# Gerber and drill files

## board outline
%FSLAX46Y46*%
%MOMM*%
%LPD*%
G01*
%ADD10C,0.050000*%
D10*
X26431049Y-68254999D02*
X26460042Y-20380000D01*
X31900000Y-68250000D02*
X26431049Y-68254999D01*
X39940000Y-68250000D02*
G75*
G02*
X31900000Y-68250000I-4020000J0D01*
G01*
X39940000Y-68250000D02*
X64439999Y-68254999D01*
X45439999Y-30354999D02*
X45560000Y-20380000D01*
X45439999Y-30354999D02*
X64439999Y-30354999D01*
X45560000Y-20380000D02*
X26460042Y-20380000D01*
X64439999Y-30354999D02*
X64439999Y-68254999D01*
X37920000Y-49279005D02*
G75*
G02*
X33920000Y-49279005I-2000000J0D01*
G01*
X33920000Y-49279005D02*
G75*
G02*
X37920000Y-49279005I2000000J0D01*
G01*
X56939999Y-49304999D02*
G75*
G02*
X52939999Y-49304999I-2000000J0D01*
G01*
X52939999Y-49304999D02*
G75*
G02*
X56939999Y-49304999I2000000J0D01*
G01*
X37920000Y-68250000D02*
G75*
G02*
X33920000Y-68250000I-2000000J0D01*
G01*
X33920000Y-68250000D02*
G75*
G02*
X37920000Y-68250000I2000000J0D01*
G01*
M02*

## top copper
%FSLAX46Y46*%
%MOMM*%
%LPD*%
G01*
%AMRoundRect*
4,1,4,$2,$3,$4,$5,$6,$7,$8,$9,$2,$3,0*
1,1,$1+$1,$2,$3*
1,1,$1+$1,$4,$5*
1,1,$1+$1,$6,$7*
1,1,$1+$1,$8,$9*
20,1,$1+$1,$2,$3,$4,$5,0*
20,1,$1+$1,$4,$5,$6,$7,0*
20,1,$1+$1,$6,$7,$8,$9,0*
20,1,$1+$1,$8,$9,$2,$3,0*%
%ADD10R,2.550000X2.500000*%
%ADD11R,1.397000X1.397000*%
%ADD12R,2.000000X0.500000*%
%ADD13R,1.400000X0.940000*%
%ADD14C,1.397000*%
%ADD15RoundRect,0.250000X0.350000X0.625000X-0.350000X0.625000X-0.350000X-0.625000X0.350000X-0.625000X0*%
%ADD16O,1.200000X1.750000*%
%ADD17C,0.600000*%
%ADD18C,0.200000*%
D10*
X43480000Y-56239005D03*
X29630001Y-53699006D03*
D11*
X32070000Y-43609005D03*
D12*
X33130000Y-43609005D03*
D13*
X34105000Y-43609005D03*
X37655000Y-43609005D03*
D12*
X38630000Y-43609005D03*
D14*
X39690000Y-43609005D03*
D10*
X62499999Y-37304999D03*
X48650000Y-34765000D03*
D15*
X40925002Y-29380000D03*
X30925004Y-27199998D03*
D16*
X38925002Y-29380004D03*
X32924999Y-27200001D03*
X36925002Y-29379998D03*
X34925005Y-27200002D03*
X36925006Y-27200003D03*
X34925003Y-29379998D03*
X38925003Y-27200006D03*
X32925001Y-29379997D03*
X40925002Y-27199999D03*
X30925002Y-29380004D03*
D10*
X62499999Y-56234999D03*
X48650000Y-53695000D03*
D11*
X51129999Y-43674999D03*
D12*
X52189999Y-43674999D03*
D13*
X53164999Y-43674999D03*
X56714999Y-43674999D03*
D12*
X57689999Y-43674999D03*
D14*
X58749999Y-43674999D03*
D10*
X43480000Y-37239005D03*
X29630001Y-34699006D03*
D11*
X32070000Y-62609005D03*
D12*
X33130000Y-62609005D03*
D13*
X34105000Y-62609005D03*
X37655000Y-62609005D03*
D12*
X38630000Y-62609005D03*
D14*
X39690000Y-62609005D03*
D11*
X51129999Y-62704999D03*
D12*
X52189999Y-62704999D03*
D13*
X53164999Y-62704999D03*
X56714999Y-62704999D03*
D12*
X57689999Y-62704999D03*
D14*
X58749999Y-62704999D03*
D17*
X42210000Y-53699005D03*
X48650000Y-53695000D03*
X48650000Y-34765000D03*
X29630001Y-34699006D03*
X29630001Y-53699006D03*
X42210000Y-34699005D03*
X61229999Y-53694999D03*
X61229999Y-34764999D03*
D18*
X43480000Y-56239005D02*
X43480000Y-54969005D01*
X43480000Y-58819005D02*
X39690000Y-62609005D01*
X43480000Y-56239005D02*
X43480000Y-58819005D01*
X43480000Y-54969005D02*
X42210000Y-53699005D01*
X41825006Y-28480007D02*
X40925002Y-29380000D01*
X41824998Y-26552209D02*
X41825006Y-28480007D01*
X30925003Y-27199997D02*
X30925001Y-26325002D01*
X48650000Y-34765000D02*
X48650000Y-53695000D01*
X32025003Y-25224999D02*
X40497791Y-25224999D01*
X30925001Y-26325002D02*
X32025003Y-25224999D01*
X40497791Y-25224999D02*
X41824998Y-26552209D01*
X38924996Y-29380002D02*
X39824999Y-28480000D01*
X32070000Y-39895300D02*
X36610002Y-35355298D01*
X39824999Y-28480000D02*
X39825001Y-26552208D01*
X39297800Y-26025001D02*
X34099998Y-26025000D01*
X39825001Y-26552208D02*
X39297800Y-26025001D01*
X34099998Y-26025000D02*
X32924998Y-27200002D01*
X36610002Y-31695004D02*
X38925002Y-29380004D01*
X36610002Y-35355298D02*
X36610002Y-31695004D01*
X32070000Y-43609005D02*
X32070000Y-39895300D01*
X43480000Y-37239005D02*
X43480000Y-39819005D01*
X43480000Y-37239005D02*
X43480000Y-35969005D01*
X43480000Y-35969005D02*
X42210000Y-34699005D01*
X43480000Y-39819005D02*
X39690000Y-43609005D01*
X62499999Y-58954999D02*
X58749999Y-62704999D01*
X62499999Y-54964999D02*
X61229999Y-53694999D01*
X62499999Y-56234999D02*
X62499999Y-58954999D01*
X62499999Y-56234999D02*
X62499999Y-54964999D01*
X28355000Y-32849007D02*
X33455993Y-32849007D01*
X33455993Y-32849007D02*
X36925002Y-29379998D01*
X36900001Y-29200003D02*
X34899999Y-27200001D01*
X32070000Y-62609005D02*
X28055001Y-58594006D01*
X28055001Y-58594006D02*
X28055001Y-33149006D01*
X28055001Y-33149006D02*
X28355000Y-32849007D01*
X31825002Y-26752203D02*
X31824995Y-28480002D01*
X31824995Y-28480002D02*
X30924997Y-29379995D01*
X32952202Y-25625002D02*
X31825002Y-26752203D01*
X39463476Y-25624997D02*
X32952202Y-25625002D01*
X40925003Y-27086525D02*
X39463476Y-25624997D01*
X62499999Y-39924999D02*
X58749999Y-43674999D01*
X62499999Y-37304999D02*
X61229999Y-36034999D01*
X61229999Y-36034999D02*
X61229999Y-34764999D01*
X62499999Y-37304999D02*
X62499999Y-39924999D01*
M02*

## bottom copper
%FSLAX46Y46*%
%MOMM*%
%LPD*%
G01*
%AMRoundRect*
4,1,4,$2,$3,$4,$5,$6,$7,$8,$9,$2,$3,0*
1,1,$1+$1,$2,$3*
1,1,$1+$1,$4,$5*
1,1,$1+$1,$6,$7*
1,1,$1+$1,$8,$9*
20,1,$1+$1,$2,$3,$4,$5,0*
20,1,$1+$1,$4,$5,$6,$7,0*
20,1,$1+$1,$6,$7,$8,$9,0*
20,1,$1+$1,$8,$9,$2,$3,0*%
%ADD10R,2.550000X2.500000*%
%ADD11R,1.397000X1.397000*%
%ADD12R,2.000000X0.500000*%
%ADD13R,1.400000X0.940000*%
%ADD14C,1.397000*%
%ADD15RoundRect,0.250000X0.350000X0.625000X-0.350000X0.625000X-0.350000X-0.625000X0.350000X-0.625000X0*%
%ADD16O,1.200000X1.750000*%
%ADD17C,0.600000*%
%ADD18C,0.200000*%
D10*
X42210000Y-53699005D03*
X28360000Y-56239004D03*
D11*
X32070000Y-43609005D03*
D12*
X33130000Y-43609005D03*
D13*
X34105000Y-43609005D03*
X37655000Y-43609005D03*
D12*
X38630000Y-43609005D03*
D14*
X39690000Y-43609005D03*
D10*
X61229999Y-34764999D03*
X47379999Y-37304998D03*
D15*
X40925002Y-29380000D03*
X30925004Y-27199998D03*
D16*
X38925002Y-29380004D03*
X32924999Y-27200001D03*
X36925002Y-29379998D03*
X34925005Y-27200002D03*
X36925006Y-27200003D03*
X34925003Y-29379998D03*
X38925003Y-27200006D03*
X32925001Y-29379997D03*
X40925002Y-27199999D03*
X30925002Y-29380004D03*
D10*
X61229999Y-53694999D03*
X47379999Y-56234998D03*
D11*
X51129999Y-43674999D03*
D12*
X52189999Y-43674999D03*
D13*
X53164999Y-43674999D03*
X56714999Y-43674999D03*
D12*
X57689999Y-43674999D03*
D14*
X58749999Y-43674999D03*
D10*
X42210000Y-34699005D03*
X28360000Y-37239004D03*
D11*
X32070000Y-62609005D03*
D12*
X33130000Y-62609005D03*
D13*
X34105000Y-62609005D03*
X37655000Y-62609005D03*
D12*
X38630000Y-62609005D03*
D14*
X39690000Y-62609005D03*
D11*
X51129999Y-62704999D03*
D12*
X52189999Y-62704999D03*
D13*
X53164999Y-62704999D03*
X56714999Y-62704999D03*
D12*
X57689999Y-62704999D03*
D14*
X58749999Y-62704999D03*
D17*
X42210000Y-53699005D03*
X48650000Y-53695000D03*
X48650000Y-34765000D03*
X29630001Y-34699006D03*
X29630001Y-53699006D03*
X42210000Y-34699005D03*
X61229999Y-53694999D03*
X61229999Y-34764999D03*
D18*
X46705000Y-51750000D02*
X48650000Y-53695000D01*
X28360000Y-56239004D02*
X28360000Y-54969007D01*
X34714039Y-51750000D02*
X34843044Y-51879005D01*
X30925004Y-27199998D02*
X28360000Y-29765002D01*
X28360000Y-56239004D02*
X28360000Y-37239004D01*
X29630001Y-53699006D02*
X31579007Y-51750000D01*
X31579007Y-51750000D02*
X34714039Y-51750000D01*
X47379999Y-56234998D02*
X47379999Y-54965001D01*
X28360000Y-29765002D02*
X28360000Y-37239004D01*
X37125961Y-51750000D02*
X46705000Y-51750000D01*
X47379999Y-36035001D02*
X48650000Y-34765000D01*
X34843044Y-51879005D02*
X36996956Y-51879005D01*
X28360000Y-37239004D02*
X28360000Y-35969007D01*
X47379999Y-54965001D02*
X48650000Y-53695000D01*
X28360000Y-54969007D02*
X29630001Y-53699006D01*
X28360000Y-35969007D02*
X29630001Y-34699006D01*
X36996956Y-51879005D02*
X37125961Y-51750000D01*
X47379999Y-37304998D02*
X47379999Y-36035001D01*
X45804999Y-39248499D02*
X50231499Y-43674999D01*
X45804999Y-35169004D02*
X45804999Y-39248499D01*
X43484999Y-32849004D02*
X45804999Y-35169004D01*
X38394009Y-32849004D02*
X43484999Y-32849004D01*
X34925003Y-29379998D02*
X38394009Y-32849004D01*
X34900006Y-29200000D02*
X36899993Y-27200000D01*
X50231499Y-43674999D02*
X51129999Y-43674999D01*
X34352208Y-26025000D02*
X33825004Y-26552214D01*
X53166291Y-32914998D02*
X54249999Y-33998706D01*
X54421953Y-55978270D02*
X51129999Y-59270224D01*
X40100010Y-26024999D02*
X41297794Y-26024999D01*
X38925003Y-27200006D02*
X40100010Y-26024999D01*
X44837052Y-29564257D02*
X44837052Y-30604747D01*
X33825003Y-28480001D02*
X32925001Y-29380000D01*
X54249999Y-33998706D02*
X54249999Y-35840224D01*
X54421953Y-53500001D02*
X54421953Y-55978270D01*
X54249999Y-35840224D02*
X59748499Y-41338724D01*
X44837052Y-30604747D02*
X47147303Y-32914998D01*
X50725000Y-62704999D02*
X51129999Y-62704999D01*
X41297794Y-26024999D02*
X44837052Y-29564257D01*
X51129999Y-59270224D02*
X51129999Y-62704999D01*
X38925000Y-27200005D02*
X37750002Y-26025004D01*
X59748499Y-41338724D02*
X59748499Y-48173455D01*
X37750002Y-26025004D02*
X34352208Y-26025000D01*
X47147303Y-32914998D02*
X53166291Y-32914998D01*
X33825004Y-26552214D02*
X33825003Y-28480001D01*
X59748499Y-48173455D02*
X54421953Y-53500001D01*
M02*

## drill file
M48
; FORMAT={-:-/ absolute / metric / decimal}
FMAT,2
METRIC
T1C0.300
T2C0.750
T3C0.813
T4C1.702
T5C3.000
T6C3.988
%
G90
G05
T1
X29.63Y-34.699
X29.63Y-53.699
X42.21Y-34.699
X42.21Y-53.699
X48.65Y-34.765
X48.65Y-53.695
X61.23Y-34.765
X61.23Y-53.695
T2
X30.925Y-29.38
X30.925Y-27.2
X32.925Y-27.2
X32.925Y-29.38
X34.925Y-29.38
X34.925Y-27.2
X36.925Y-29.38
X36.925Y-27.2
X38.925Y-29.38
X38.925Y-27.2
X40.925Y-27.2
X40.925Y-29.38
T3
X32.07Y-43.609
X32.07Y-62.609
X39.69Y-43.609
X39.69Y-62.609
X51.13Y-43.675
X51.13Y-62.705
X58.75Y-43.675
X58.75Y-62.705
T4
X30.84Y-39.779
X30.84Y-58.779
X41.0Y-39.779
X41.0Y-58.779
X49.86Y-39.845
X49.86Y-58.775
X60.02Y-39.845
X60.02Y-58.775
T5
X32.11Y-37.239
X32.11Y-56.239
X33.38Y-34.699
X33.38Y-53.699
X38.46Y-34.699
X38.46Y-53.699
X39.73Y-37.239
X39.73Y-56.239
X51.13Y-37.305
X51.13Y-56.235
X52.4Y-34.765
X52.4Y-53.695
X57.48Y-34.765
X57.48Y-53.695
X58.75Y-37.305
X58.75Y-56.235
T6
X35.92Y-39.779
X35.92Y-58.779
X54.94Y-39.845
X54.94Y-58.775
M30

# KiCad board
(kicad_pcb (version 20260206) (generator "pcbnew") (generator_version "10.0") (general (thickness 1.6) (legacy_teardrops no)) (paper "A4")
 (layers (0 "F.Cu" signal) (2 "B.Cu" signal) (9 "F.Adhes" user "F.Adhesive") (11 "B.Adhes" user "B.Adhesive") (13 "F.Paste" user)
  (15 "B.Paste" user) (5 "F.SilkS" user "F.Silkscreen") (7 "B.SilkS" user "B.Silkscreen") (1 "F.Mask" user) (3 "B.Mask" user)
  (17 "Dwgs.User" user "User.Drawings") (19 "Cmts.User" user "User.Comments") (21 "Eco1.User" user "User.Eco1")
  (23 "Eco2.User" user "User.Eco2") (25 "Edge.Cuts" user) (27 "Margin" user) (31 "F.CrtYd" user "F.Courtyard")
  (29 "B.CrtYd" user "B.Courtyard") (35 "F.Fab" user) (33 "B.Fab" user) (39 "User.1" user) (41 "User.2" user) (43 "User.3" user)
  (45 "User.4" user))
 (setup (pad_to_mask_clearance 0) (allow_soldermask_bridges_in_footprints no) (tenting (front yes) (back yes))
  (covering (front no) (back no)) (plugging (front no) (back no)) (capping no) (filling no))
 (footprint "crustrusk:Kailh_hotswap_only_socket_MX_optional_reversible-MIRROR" (layer "F.Cu") (at 35.92 58.779005)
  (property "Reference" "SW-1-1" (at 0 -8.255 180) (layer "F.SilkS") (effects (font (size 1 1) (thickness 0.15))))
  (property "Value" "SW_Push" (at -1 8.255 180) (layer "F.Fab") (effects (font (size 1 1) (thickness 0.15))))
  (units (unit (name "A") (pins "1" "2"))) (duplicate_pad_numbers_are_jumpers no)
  (pad "" np_thru_hole circle (at -5.08 0) (size 1.7018 1.7018) (drill 1.7018) (layers "*.Cu" "*.Mask"))
  (pad "" np_thru_hole circle (at -3.81 -2.54 180) (size 3 3) (drill 3) (layers "*.Cu" "*.Mask"))
  (pad "" np_thru_hole circle (at -2.54 -5.079998) (size 3 3) (drill 3) (layers "*.Cu" "*.Mask"))
  (pad "" np_thru_hole circle (at 0 0) (size 3.9878 3.9878) (drill 3.9878) (layers "*.Cu" "*.Mask"))
  (pad "" np_thru_hole circle (at 2.540002 -5.080001 180) (size 3 3) (drill 3) (layers "*.Cu" "*.Mask"))
  (pad "" np_thru_hole circle (at 3.81 -2.54) (size 3 3) (drill 3) (layers "*.Cu" "*.Mask"))
  (pad "" np_thru_hole circle (at 5.08 0) (size 1.7018 1.7018) (drill 1.7018) (layers "*.Cu" "*.Mask"))
  (pad "1" smd rect (at 6.29 -5.08 180) (size 2.55 2.5) (layers "B.Cu" "B.Mask" "B.Paste") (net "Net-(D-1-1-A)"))
  (pad "1" smd rect (at 7.56 -2.54) (size 2.55 2.5) (layers "F.Cu" "F.Mask" "F.Paste") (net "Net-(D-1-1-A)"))
  (pad "2" smd rect (at -7.56 -2.540001 180) (size 2.55 2.5) (layers "B.Cu" "B.Mask" "B.Paste") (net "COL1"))
  (pad "2" smd rect (at -6.289999 -5.079999) (size 2.55 2.5) (layers "F.Cu" "F.Mask" "F.Paste") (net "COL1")))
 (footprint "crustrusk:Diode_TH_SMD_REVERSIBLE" (layer "F.Cu") (at 35.88 43.609005)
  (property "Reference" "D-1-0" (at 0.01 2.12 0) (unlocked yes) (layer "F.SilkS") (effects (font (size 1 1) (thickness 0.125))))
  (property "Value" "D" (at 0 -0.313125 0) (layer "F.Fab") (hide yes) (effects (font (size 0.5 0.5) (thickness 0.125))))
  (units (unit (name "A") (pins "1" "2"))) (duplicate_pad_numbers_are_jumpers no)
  (pad "1" thru_hole rect (at -3.81 0) (size 1.397 1.397) (drill 0.8128) (layers "*.Cu" "*.Mask") (remove_unused_layers no) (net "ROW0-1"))
  (pad "1" smd rect (at -2.75 0 180) (size 2 0.5) (layers "F.Cu") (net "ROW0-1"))
  (pad "1" smd rect (at -2.75 0) (size 2 0.5) (layers "B.Cu") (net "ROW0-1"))
  (pad "1" smd rect (at -1.775 0 180) (size 1.4 0.94) (layers "F.Cu" "F.Mask" "F.Paste") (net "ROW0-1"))
  (pad "1" smd rect (at -1.775 0) (size 1.4 0.94) (layers "B.Cu" "B.Mask" "B.Paste") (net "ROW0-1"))
  (pad "2" smd rect (at 1.775 0 180) (size 1.4 0.94) (layers "F.Cu" "F.Mask" "F.Paste") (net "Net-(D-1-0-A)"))
  (pad "2" smd rect (at 1.775 0) (size 1.4 0.94) (layers "B.Cu" "B.Mask" "B.Paste") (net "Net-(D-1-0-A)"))
  (pad "2" smd rect (at 2.75 0 180) (size 2 0.5) (layers "F.Cu") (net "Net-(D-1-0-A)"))
  (pad "2" smd rect (at 2.75 0) (size 2 0.5) (layers "B.Cu") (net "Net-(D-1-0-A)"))
  (pad "2" thru_hole circle (at 3.81 0) (size 1.397 1.397) (drill 0.8128) (layers "*.Cu" "*.Mask") (remove_unused_layers no)
   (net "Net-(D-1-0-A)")))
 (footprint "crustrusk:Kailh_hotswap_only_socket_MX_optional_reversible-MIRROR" (layer "F.Cu") (at 54.939999 39.844999)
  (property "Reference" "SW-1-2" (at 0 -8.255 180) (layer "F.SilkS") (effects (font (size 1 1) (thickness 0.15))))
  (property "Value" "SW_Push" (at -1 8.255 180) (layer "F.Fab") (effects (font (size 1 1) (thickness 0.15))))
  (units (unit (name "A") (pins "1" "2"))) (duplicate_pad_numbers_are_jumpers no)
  (pad "" np_thru_hole circle (at -5.08 0) (size 1.7018 1.7018) (drill 1.7018) (layers "*.Cu" "*.Mask"))
  (pad "" np_thru_hole circle (at -3.81 -2.54 180) (size 3 3) (drill 3) (layers "*.Cu" "*.Mask"))
  (pad "" np_thru_hole circle (at -2.54 -5.079998) (size 3 3) (drill 3) (layers "*.Cu" "*.Mask"))
  (pad "" np_thru_hole circle (at 0 0) (size 3.9878 3.9878) (drill 3.9878) (layers "*.Cu" "*.Mask"))
  (pad "" np_thru_hole circle (at 2.540002 -5.080001 180) (size 3 3) (drill 3) (layers "*.Cu" "*.Mask"))
  (pad "" np_thru_hole circle (at 3.81 -2.54) (size 3 3) (drill 3) (layers "*.Cu" "*.Mask"))
  (pad "" np_thru_hole circle (at 5.08 0) (size 1.7018 1.7018) (drill 1.7018) (layers "*.Cu" "*.Mask"))
  (pad "1" smd rect (at 6.29 -5.08 180) (size 2.55 2.5) (layers "B.Cu" "B.Mask" "B.Paste") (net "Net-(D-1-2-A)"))
  (pad "1" smd rect (at 7.56 -2.54) (size 2.55 2.5) (layers "F.Cu" "F.Mask" "F.Paste") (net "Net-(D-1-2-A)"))
  (pad "2" smd rect (at -7.56 -2.540001 180) (size 2.55 2.5) (layers "B.Cu" "B.Mask" "B.Paste") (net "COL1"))
  (pad "2" smd rect (at -6.289999 -5.079999) (size 2.55 2.5) (layers "F.Cu" "F.Mask" "F.Paste") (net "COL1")))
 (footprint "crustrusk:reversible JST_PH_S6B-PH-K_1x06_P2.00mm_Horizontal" (layer "F.Cu") (at 40.925002 29.38 180)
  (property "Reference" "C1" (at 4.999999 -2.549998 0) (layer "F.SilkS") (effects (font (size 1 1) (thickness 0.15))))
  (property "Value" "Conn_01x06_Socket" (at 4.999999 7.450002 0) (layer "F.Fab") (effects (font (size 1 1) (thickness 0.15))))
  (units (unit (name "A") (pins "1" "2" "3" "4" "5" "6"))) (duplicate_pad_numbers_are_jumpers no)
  (pad "1" thru_hole roundrect (at 0 0 180) (size 1.2 1.75) (drill 0.75) (layers "*.Cu" "*.Mask") (remove_unused_layers no)
   (roundrect_rratio 0.208333) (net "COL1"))
  (pad "1" thru_hole roundrect (at 9.999998 2.180002 180) (size 1.2 1.75) (drill 0.75) (layers "*.Cu" "*.Mask") (remove_unused_layers no)
   (roundrect_rratio 0.208333) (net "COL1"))
  (pad "2" thru_hole oval (at 2 -0.000004 180) (size 1.2 1.75) (drill 0.75) (layers "*.Cu" "*.Mask") (remove_unused_layers no)
   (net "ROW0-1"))
  (pad "2" thru_hole oval (at 8.000003 2.179999 180) (size 1.2 1.75) (drill 0.75) (layers "*.Cu" "*.Mask") (remove_unused_layers no)
   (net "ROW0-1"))
  (pad "3" thru_hole oval (at 4 0.000002 180) (size 1.2 1.75) (drill 0.75) (layers "*.Cu" "*.Mask") (remove_unused_layers no) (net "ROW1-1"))
  (pad "3" thru_hole oval (at 5.999997 2.179998 180) (size 1.2 1.75) (drill 0.75) (layers "*.Cu" "*.Mask") (remove_unused_layers no)
   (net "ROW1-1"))
  (pad "4" thru_hole oval (at 3.999996 2.179997 180) (size 1.2 1.75) (drill 0.75) (layers "*.Cu" "*.Mask") (remove_unused_layers no)
   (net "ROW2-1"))
  (pad "4" thru_hole oval (at 5.999999 0.000002 180) (size 1.2 1.75) (drill 0.75) (layers "*.Cu" "*.Mask") (remove_unused_layers no)
   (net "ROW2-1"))
  (pad "5" thru_hole oval (at 1.999999 2.179994 180) (size 1.2 1.75) (drill 0.75) (layers "*.Cu" "*.Mask") (remove_unused_layers no)
   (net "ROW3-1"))
  (pad "5" thru_hole oval (at 8.000001 0.000003 180) (size 1.2 1.75) (drill 0.75) (layers "*.Cu" "*.Mask") (remove_unused_layers no)
   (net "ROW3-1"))
  (pad "6" thru_hole oval (at 0 2.180001 180) (size 1.2 1.75) (drill 0.75) (layers "*.Cu" "*.Mask") (remove_unused_layers no) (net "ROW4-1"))
  (pad "6" thru_hole oval (at 10 -0.000004 180) (size 1.2 1.75) (drill 0.75) (layers "*.Cu" "*.Mask") (remove_unused_layers no)
   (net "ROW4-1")))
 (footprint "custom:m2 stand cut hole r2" (layer "F.Cu") (at 35.92 49.279005)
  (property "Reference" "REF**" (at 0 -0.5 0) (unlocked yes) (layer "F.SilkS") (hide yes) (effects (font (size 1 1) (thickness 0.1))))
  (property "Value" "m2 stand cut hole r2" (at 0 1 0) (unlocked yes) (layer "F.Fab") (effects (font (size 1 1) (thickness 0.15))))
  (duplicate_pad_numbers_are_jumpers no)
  (fp_circle (center 0 0) (end 2 0) (stroke (width 0.05) (type default)) (fill no) (layer "Edge.Cuts")))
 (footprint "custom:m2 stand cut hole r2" (layer "F.Cu") (at 54.939999 49.304999)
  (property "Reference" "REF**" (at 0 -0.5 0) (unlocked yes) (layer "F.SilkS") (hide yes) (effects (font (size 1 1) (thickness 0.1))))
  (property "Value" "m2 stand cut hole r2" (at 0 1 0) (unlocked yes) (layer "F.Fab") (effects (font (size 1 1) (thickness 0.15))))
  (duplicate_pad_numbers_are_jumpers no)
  (fp_circle (center 0 0) (end 2 0) (stroke (width 0.05) (type default)) (fill no) (layer "Edge.Cuts")))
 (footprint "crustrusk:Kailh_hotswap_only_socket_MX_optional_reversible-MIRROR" (layer "F.Cu") (at 54.939999 58.774999)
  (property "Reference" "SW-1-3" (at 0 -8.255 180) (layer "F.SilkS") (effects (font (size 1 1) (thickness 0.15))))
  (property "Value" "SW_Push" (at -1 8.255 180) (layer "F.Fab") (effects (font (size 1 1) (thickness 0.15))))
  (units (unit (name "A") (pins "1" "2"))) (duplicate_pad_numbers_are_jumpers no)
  (pad "" np_thru_hole circle (at -5.08 0) (size 1.7018 1.7018) (drill 1.7018) (layers "*.Cu" "*.Mask"))
  (pad "" np_thru_hole circle (at -3.81 -2.54 180) (size 3 3) (drill 3) (layers "*.Cu" "*.Mask"))
  (pad "" np_thru_hole circle (at -2.54 -5.079998) (size 3 3) (drill 3) (layers "*.Cu" "*.Mask"))
  (pad "" np_thru_hole circle (at 0 0) (size 3.9878 3.9878) (drill 3.9878) (layers "*.Cu" "*.Mask"))
  (pad "" np_thru_hole circle (at 2.540002 -5.080001 180) (size 3 3) (drill 3) (layers "*.Cu" "*.Mask"))
  (pad "" np_thru_hole circle (at 3.81 -2.54) (size 3 3) (drill 3) (layers "*.Cu" "*.Mask"))
  (pad "" np_thru_hole circle (at 5.08 0) (size 1.7018 1.7018) (drill 1.7018) (layers "*.Cu" "*.Mask"))
  (pad "1" smd rect (at 6.29 -5.08 180) (size 2.55 2.5) (layers "B.Cu" "B.Mask" "B.Paste") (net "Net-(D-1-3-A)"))
  (pad "1" smd rect (at 7.56 -2.54) (size 2.55 2.5) (layers "F.Cu" "F.Mask" "F.Paste") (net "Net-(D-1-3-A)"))
  (pad "2" smd rect (at -7.56 -2.540001 180) (size 2.55 2.5) (layers "B.Cu" "B.Mask" "B.Paste") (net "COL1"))
  (pad "2" smd rect (at -6.289999 -5.079999) (size 2.55 2.5) (layers "F.Cu" "F.Mask" "F.Paste") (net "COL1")))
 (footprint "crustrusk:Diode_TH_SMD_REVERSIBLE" (layer "F.Cu") (at 54.939999 43.674999)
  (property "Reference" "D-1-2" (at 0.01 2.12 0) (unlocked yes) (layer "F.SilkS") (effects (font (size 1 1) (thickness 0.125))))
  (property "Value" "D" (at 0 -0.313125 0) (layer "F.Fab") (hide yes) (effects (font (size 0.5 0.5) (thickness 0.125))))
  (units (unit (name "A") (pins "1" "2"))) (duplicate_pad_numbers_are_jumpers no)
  (pad "1" thru_hole rect (at -3.81 0) (size 1.397 1.397) (drill 0.8128) (layers "*.Cu" "*.Mask") (remove_unused_layers no) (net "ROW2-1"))
  (pad "1" smd rect (at -2.75 0 180) (size 2 0.5) (layers "F.Cu") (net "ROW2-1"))
  (pad "1" smd rect (at -2.75 0) (size 2 0.5) (layers "B.Cu") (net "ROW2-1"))
  (pad "1" smd rect (at -1.775 0 180) (size 1.4 0.94) (layers "F.Cu" "F.Mask" "F.Paste") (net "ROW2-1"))
  (pad "1" smd rect (at -1.775 0) (size 1.4 0.94) (layers "B.Cu" "B.Mask" "B.Paste") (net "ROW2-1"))
  (pad "2" smd rect (at 1.775 0 180) (size 1.4 0.94) (layers "F.Cu" "F.Mask" "F.Paste") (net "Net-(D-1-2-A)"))
  (pad "2" smd rect (at 1.775 0) (size 1.4 0.94) (layers "B.Cu" "B.Mask" "B.Paste") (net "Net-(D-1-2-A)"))
  (pad "2" smd rect (at 2.75 0 180) (size 2 0.5) (layers "F.Cu") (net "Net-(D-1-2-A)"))
  (pad "2" smd rect (at 2.75 0) (size 2 0.5) (layers "B.Cu") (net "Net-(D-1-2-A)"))
  (pad "2" thru_hole circle (at 3.81 0) (size 1.397 1.397) (drill 0.8128) (layers "*.Cu" "*.Mask") (remove_unused_layers no)
   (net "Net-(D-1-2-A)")))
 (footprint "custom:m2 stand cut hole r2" (layer "F.Cu") (at 35.92 68.25)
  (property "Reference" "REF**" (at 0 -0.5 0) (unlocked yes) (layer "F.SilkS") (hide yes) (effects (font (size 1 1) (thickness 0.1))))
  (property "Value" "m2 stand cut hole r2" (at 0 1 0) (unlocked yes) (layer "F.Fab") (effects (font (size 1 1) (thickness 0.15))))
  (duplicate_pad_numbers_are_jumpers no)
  (fp_circle (center 0 0) (end 2 0) (stroke (width 0.05) (type default)) (fill no) (layer "Edge.Cuts")))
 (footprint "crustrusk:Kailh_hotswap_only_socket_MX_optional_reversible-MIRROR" (layer "F.Cu") (at 35.92 39.779005)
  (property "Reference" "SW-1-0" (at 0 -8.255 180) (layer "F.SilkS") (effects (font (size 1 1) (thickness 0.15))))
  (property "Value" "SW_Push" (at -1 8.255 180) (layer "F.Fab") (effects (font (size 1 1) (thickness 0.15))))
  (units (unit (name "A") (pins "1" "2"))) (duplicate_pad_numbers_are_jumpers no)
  (pad "" np_thru_hole circle (at -5.08 0) (size 1.7018 1.7018) (drill 1.7018) (layers "*.Cu" "*.Mask"))
  (pad "" np_thru_hole circle (at -3.81 -2.54 180) (size 3 3) (drill 3) (layers "*.Cu" "*.Mask"))
  (pad "" np_thru_hole circle (at -2.54 -5.079998) (size 3 3) (drill 3) (layers "*.Cu" "*.Mask"))
  (pad "" np_thru_hole circle (at 0 0) (size 3.9878 3.9878) (drill 3.9878) (layers "*.Cu" "*.Mask"))
  (pad "" np_thru_hole circle (at 2.540002 -5.080001 180) (size 3 3) (drill 3) (layers "*.Cu" "*.Mask"))
  (pad "" np_thru_hole circle (at 3.81 -2.54) (size 3 3) (drill 3) (layers "*.Cu" "*.Mask"))
  (pad "" np_thru_hole circle (at 5.08 0) (size 1.7018 1.7018) (drill 1.7018) (layers "*.Cu" "*.Mask"))
  (pad "1" smd rect (at 6.29 -5.08 180) (size 2.55 2.5) (layers "B.Cu" "B.Mask" "B.Paste") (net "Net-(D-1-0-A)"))
  (pad "1" smd rect (at 7.56 -2.54) (size 2.55 2.5) (layers "F.Cu" "F.Mask" "F.Paste") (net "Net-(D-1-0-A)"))
  (pad "2" smd rect (at -7.56 -2.540001 180) (size 2.55 2.5) (layers "B.Cu" "B.Mask" "B.Paste") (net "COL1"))
  (pad "2" smd rect (at -6.289999 -5.079999) (size 2.55 2.5) (layers "F.Cu" "F.Mask" "F.Paste") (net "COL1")))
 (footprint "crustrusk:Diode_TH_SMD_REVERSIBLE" (layer "F.Cu") (at 35.88 62.609005)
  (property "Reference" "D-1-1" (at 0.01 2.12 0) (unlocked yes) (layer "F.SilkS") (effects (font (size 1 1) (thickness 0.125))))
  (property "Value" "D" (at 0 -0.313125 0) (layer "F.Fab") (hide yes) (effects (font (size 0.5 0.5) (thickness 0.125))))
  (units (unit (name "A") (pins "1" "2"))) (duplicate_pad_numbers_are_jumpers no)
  (pad "1" thru_hole rect (at -3.81 0) (size 1.397 1.397) (drill 0.8128) (layers "*.Cu" "*.Mask") (remove_unused_layers no) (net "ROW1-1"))
  (pad "1" smd rect (at -2.75 0 180) (size 2 0.5) (layers "F.Cu") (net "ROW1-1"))
  (pad "1" smd rect (at -2.75 0) (size 2 0.5) (layers "B.Cu") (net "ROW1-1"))
  (pad "1" smd rect (at -1.775 0 180) (size 1.4 0.94) (layers "F.Cu" "F.Mask" "F.Paste") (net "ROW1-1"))
  (pad "1" smd rect (at -1.775 0) (size 1.4 0.94) (layers "B.Cu" "B.Mask" "B.Paste") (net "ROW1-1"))
  (pad "2" smd rect (at 1.775 0 180) (size 1.4 0.94) (layers "F.Cu" "F.Mask" "F.Paste") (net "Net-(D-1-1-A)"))
  (pad "2" smd rect (at 1.775 0) (size 1.4 0.94) (layers "B.Cu" "B.Mask" "B.Paste") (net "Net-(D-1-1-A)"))
  (pad "2" smd rect (at 2.75 0 180) (size 2 0.5) (layers "F.Cu") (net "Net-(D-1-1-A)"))
  (pad "2" smd rect (at 2.75 0) (size 2 0.5) (layers "B.Cu") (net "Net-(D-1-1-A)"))
  (pad "2" thru_hole circle (at 3.81 0) (size 1.397 1.397) (drill 0.8128) (layers "*.Cu" "*.Mask") (remove_unused_layers no)
   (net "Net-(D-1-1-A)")))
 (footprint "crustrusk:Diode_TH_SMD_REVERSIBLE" (layer "F.Cu") (at 54.939999 62.704999)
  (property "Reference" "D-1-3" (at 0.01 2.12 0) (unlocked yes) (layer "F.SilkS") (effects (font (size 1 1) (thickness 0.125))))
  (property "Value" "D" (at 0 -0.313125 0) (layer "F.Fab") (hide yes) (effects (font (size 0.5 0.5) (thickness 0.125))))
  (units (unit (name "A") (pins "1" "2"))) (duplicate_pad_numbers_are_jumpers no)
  (pad "1" thru_hole rect (at -3.81 0) (size 1.397 1.397) (drill 0.8128) (layers "*.Cu" "*.Mask") (remove_unused_layers no) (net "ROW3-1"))
  (pad "1" smd rect (at -2.75 0 180) (size 2 0.5) (layers "F.Cu") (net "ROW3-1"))
  (pad "1" smd rect (at -2.75 0) (size 2 0.5) (layers "B.Cu") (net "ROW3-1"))
  (pad "1" smd rect (at -1.775 0 180) (size 1.4 0.94) (layers "F.Cu" "F.Mask" "F.Paste") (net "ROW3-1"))
  (pad "1" smd rect (at -1.775 0) (size 1.4 0.94) (layers "B.Cu" "B.Mask" "B.Paste") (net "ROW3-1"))
  (pad "2" smd rect (at 1.775 0 180) (size 1.4 0.94) (layers "F.Cu" "F.Mask" "F.Paste") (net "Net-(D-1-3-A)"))
  (pad "2" smd rect (at 1.775 0) (size 1.4 0.94) (layers "B.Cu" "B.Mask" "B.Paste") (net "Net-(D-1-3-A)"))
  (pad "2" smd rect (at 2.75 0 180) (size 2 0.5) (layers "F.Cu") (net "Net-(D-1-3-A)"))
  (pad "2" smd rect (at 2.75 0) (size 2 0.5) (layers "B.Cu") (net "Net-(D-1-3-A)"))
  (pad "2" thru_hole circle (at 3.81 0) (size 1.397 1.397) (drill 0.8128) (layers "*.Cu" "*.Mask") (remove_unused_layers no)
   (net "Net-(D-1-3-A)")))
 (gr_line (start 26.431049 68.254999) (end 26.460042 20.38) (stroke (width 0.05) (type default)) (layer "Edge.Cuts"))
 (gr_line (start 31.9 68.25) (end 26.431049 68.254999) (stroke (width 0.05) (type default)) (layer "Edge.Cuts"))
 (gr_arc (start 39.94 68.25) (mid 35.92 72.27) (end 31.9 68.25) (stroke (width 0.05) (type default)) (layer "Edge.Cuts"))
 (gr_line (start 39.94 68.25) (end 64.439999 68.254999) (stroke (width 0.05) (type default)) (layer "Edge.Cuts"))
 (gr_line (start 45.439999 30.354999) (end 45.56 20.38) (stroke (width 0.05) (type default)) (layer "Edge.Cuts"))
 (gr_line (start 45.439999 30.354999) (end 64.439999 30.354999) (stroke (width 0.05) (type default)) (layer "Edge.Cuts"))
 (gr_line (start 45.56 20.38) (end 26.460042 20.38) (stroke (width 0.05) (type default)) (layer "Edge.Cuts"))
 (gr_line (start 64.439999 30.354999) (end 64.439999 68.254999) (stroke (width 0.05) (type default)) (layer "Edge.Cuts"))
 (segment (start 43.48 56.239005) (end 43.48 54.969005) (width 0.2) (layer "F.Cu") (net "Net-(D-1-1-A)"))
 (segment (start 43.48 58.819005) (end 39.69 62.609005) (width 0.2) (layer "F.Cu") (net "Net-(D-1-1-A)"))
 (segment (start 43.48 56.239005) (end 43.48 58.819005) (width 0.2) (layer "F.Cu") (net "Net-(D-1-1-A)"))
 (segment (start 43.48 54.969005) (end 42.21 53.699005) (width 0.2) (layer "F.Cu") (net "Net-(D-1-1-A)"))
 (via (at 42.21 53.699005) (size 0.6) (drill 0.3) (layers "F.Cu" "B.Cu") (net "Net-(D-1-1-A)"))
 (segment (start 41.825006 28.480007) (end 40.925002 29.38) (width 0.2) (layer "F.Cu") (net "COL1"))
 (segment (start 41.824998 26.552209) (end 41.825006 28.480007) (width 0.2) (layer "F.Cu") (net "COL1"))
 (segment (start 30.925003 27.199997) (end 30.925001 26.325002) (width 0.2) (layer "F.Cu") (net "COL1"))
 (segment (start 48.65 34.765) (end 48.65 53.695) (width 0.2) (layer "F.Cu") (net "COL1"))
 (segment (start 32.025003 25.224999) (end 40.497791 25.224999) (width 0.2) (layer "F.Cu") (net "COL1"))
 (segment (start 30.925001 26.325002) (end 32.025003 25.224999) (width 0.2) (layer "F.Cu") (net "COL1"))
 (segment (start 40.497791 25.224999) (end 41.824998 26.552209) (width 0.2) (layer "F.Cu") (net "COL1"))
 (via (at 48.65 53.695) (size 0.6) (drill 0.3) (layers "F.Cu" "B.Cu") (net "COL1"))
 (via (at 48.65 34.765) (size 0.6) (drill 0.3) (layers "F.Cu" "B.Cu") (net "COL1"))
 (via (at 29.630001 34.699006) (size 0.6) (drill 0.3) (layers "F.Cu" "B.Cu") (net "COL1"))
 (via (at 29.630001 53.699006) (size 0.6) (drill 0.3) (layers "F.Cu" "B.Cu") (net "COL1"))
 (segment (start 46.705 51.75) (end 48.65 53.695) (width 0.2) (layer "B.Cu") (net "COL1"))
 (segment (start 28.36 56.239004) (end 28.36 54.969007) (width 0.2) (layer "B.Cu") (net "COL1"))
 (segment (start 34.714039 51.75) (end 34.843044 51.879005) (width 0.2) (layer "B.Cu") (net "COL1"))
 (segment (start 30.925004 27.199998) (end 28.36 29.765002) (width 0.2) (layer "B.Cu") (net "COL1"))
 (segment (start 28.36 56.239004) (end 28.36 37.239004) (width 0.2) (layer "B.Cu") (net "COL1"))
 (segment (start 29.630001 53.699006) (end 31.579007 51.75) (width 0.2) (layer "B.Cu") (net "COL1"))
 (segment (start 31.579007 51.75) (end 34.714039 51.75) (width 0.2) (layer "B.Cu") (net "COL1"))
 (segment (start 47.379999 56.234998) (end 47.379999 54.965001) (width 0.2) (layer "B.Cu") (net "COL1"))
 (segment (start 28.36 29.765002) (end 28.36 37.239004) (width 0.2) (layer "B.Cu") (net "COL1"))
 (segment (start 37.125961 51.75) (end 46.705 51.75) (width 0.2) (layer "B.Cu") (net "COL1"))
 (segment (start 47.379999 36.035001) (end 48.65 34.765) (width 0.2) (layer "B.Cu") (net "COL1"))
 (segment (start 34.843044 51.879005) (end 36.996956 51.879005) (width 0.2) (layer "B.Cu") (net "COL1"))
 (segment (start 28.36 37.239004) (end 28.36 35.969007) (width 0.2) (layer "B.Cu") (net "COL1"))
 (segment (start 47.379999 54.965001) (end 48.65 53.695) (width 0.2) (layer "B.Cu") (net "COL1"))
 (segment (start 28.36 54.969007) (end 29.630001 53.699006) (width 0.2) (layer "B.Cu") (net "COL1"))
 (segment (start 28.36 35.969007) (end 29.630001 34.699006) (width 0.2) (layer "B.Cu") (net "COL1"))
 (segment (start 36.996956 51.879005) (end 37.125961 51.75) (width 0.2) (layer "B.Cu") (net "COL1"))
 (segment (start 47.379999 37.304998) (end 47.379999 36.035001) (width 0.2) (layer "B.Cu") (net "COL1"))
 (segment (start 38.924996 29.380002) (end 39.824999 28.48) (width 0.2) (layer "F.Cu") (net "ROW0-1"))
 (segment (start 32.07 39.8953) (end 36.610002 35.355298) (width 0.2) (layer "F.Cu") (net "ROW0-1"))
 (segment (start 39.824999 28.48) (end 39.825001 26.552208) (width 0.2) (layer "F.Cu") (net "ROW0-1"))
 (segment (start 39.2978 26.025001) (end 34.099998 26.025) (width 0.2) (layer "F.Cu") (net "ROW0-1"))
 (segment (start 39.825001 26.552208) (end 39.2978 26.025001) (width 0.2) (layer "F.Cu") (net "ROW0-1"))
 (segment (start 34.099998 26.025) (end 32.924998 27.200002) (width 0.2) (layer "F.Cu") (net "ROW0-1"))
 (segment (start 36.610002 31.695004) (end 38.925002 29.380004) (width 0.2) (layer "F.Cu") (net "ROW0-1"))
 (segment (start 36.610002 35.355298) (end 36.610002 31.695004) (width 0.2) (layer "F.Cu") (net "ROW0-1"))
 (segment (start 32.07 43.609005) (end 32.07 39.8953) (width 0.2) (layer "F.Cu") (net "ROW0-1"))
 (segment (start 43.48 37.239005) (end 43.48 39.819005) (width 0.2) (layer "F.Cu") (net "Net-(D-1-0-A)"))
 (segment (start 43.48 37.239005) (end 43.48 35.969005) (width 0.2) (layer "F.Cu") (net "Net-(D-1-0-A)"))
 (segment (start 43.48 35.969005) (end 42.21 34.699005) (width 0.2) (layer "F.Cu") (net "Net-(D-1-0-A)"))
 (segment (start 43.48 39.819005) (end 39.69 43.609005) (width 0.2) (layer "F.Cu") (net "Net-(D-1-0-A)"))
 (via (at 42.21 34.699005) (size 0.6) (drill 0.3) (layers "F.Cu" "B.Cu") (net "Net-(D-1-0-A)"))
 (segment (start 62.499999 58.954999) (end 58.749999 62.704999) (width 0.2) (layer "F.Cu") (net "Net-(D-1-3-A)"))
 (segment (start 62.499999 54.964999) (end 61.229999 53.694999) (width 0.2) (layer "F.Cu") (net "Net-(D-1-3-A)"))
 (segment (start 62.499999 56.234999) (end 62.499999 58.954999) (width 0.2) (layer "F.Cu") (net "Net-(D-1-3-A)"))
 (segment (start 62.499999 56.234999) (end 62.499999 54.964999) (width 0.2) (layer "F.Cu") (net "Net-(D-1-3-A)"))
 (via (at 61.229999 53.694999) (size 0.6) (drill 0.3) (layers "F.Cu" "B.Cu") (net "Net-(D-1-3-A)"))
 (segment (start 28.355 32.849007) (end 33.455993 32.849007) (width 0.2) (layer "F.Cu") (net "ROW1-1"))
 (segment (start 33.455993 32.849007) (end 36.925002 29.379998) (width 0.2) (layer "F.Cu") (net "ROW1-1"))
 (segment (start 36.900001 29.200003) (end 34.899999 27.200001) (width 0.2) (layer "F.Cu") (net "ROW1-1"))
 (segment (start 32.07 62.609005) (end 28.055001 58.594006) (width 0.2) (layer "F.Cu") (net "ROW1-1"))
 (segment (start 28.055001 58.594006) (end 28.055001 33.149006) (width 0.2) (layer "F.Cu") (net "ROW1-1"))
 (segment (start 28.055001 33.149006) (end 28.355 32.849007) (width 0.2) (layer "F.Cu") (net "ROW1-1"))
 (segment (start 45.804999 39.248499) (end 50.231499 43.674999) (width 0.2) (layer "B.Cu") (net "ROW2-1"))
 (segment (start 45.804999 35.169004) (end 45.804999 39.248499) (width 0.2) (layer "B.Cu") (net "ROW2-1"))
 (segment (start 43.484999 32.849004) (end 45.804999 35.169004) (width 0.2) (layer "B.Cu") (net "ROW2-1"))
 (segment (start 38.394009 32.849004) (end 43.484999 32.849004) (width 0.2) (layer "B.Cu") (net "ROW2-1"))
 (segment (start 34.925003 29.379998) (end 38.394009 32.849004) (width 0.2) (layer "B.Cu") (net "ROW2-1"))
 (segment (start 34.900006 29.2) (end 36.899993 27.2) (width 0.2) (layer "B.Cu") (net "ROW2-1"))
 (segment (start 50.231499 43.674999) (end 51.129999 43.674999) (width 0.2) (layer "B.Cu") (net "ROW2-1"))
 (segment (start 34.352208 26.025) (end 33.825004 26.552214) (width 0.2) (layer "B.Cu") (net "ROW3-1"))
 (segment (start 53.166291 32.914998) (end 54.249999 33.998706) (width 0.2) (layer "B.Cu") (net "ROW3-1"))
 (segment (start 54.421953 55.97827) (end 51.129999 59.270224) (width 0.2) (layer "B.Cu") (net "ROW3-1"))
 (segment (start 40.10001 26.024999) (end 41.297794 26.024999) (width 0.2) (layer "B.Cu") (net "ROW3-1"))
 (segment (start 38.925003 27.200006) (end 40.10001 26.024999) (width 0.2) (layer "B.Cu") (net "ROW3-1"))
 (segment (start 44.837052 29.564257) (end 44.837052 30.604747) (width 0.2) (layer "B.Cu") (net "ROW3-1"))
 (segment (start 33.825003 28.480001) (end 32.925001 29.38) (width 0.2) (layer "B.Cu") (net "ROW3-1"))
 (segment (start 54.249999 33.998706) (end 54.249999 35.840224) (width 0.2) (layer "B.Cu") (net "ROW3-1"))
 (segment (start 54.421953 53.500001) (end 54.421953 55.97827) (width 0.2) (layer "B.Cu") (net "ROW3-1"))
 (segment (start 54.249999 35.840224) (end 59.748499 41.338724) (width 0.2) (layer "B.Cu") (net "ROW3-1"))
 (segment (start 44.837052 30.604747) (end 47.147303 32.914998) (width 0.2) (layer "B.Cu") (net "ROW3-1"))
 (segment (start 50.725 62.704999) (end 51.129999 62.704999) (width 0.2) (layer "B.Cu") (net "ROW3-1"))
 (segment (start 41.297794 26.024999) (end 44.837052 29.564257) (width 0.2) (layer "B.Cu") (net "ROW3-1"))
 (segment (start 51.129999 59.270224) (end 51.129999 62.704999) (width 0.2) (layer "B.Cu") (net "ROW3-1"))
 (segment (start 38.925 27.200005) (end 37.750002 26.025004) (width 0.2) (layer "B.Cu") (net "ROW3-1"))
 (segment (start 59.748499 41.338724) (end 59.748499 48.173455) (width 0.2) (layer "B.Cu") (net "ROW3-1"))
 (segment (start 37.750002 26.025004) (end 34.352208 26.025) (width 0.2) (layer "B.Cu") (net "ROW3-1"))
 (segment (start 47.147303 32.914998) (end 53.166291 32.914998) (width 0.2) (layer "B.Cu") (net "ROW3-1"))
 (segment (start 33.825004 26.552214) (end 33.825003 28.480001) (width 0.2) (layer "B.Cu") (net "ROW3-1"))
 (segment (start 59.748499 48.173455) (end 54.421953 53.500001) (width 0.2) (layer "B.Cu") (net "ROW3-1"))
 (segment (start 31.825002 26.752203) (end 31.824995 28.480002) (width 0.2) (layer "F.Cu") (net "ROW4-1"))
 (segment (start 31.824995 28.480002) (end 30.924997 29.379995) (width 0.2) (layer "F.Cu") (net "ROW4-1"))
 (segment (start 32.952202 25.625002) (end 31.825002 26.752203) (width 0.2) (layer "F.Cu") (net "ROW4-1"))
 (segment (start 39.463476 25.624997) (end 32.952202 25.625002) (width 0.2) (layer "F.Cu") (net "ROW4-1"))
 (segment (start 40.925003 27.086525) (end 39.463476 25.624997) (width 0.2) (layer "F.Cu") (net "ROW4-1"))
 (segment (start 62.499999 39.924999) (end 58.749999 43.674999) (width 0.2) (layer "F.Cu") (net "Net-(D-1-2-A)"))
 (segment (start 62.499999 37.304999) (end 61.229999 36.034999) (width 0.2) (layer "F.Cu") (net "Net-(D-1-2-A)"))
 (segment (start 61.229999 36.034999) (end 61.229999 34.764999) (width 0.2) (layer "F.Cu") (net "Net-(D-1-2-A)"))
 (segment (start 62.499999 37.304999) (end 62.499999 39.924999) (width 0.2) (layer "F.Cu") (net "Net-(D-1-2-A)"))
 (via (at 61.229999 34.764999) (size 0.6) (drill 0.3) (layers "F.Cu" "B.Cu") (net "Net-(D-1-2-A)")))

